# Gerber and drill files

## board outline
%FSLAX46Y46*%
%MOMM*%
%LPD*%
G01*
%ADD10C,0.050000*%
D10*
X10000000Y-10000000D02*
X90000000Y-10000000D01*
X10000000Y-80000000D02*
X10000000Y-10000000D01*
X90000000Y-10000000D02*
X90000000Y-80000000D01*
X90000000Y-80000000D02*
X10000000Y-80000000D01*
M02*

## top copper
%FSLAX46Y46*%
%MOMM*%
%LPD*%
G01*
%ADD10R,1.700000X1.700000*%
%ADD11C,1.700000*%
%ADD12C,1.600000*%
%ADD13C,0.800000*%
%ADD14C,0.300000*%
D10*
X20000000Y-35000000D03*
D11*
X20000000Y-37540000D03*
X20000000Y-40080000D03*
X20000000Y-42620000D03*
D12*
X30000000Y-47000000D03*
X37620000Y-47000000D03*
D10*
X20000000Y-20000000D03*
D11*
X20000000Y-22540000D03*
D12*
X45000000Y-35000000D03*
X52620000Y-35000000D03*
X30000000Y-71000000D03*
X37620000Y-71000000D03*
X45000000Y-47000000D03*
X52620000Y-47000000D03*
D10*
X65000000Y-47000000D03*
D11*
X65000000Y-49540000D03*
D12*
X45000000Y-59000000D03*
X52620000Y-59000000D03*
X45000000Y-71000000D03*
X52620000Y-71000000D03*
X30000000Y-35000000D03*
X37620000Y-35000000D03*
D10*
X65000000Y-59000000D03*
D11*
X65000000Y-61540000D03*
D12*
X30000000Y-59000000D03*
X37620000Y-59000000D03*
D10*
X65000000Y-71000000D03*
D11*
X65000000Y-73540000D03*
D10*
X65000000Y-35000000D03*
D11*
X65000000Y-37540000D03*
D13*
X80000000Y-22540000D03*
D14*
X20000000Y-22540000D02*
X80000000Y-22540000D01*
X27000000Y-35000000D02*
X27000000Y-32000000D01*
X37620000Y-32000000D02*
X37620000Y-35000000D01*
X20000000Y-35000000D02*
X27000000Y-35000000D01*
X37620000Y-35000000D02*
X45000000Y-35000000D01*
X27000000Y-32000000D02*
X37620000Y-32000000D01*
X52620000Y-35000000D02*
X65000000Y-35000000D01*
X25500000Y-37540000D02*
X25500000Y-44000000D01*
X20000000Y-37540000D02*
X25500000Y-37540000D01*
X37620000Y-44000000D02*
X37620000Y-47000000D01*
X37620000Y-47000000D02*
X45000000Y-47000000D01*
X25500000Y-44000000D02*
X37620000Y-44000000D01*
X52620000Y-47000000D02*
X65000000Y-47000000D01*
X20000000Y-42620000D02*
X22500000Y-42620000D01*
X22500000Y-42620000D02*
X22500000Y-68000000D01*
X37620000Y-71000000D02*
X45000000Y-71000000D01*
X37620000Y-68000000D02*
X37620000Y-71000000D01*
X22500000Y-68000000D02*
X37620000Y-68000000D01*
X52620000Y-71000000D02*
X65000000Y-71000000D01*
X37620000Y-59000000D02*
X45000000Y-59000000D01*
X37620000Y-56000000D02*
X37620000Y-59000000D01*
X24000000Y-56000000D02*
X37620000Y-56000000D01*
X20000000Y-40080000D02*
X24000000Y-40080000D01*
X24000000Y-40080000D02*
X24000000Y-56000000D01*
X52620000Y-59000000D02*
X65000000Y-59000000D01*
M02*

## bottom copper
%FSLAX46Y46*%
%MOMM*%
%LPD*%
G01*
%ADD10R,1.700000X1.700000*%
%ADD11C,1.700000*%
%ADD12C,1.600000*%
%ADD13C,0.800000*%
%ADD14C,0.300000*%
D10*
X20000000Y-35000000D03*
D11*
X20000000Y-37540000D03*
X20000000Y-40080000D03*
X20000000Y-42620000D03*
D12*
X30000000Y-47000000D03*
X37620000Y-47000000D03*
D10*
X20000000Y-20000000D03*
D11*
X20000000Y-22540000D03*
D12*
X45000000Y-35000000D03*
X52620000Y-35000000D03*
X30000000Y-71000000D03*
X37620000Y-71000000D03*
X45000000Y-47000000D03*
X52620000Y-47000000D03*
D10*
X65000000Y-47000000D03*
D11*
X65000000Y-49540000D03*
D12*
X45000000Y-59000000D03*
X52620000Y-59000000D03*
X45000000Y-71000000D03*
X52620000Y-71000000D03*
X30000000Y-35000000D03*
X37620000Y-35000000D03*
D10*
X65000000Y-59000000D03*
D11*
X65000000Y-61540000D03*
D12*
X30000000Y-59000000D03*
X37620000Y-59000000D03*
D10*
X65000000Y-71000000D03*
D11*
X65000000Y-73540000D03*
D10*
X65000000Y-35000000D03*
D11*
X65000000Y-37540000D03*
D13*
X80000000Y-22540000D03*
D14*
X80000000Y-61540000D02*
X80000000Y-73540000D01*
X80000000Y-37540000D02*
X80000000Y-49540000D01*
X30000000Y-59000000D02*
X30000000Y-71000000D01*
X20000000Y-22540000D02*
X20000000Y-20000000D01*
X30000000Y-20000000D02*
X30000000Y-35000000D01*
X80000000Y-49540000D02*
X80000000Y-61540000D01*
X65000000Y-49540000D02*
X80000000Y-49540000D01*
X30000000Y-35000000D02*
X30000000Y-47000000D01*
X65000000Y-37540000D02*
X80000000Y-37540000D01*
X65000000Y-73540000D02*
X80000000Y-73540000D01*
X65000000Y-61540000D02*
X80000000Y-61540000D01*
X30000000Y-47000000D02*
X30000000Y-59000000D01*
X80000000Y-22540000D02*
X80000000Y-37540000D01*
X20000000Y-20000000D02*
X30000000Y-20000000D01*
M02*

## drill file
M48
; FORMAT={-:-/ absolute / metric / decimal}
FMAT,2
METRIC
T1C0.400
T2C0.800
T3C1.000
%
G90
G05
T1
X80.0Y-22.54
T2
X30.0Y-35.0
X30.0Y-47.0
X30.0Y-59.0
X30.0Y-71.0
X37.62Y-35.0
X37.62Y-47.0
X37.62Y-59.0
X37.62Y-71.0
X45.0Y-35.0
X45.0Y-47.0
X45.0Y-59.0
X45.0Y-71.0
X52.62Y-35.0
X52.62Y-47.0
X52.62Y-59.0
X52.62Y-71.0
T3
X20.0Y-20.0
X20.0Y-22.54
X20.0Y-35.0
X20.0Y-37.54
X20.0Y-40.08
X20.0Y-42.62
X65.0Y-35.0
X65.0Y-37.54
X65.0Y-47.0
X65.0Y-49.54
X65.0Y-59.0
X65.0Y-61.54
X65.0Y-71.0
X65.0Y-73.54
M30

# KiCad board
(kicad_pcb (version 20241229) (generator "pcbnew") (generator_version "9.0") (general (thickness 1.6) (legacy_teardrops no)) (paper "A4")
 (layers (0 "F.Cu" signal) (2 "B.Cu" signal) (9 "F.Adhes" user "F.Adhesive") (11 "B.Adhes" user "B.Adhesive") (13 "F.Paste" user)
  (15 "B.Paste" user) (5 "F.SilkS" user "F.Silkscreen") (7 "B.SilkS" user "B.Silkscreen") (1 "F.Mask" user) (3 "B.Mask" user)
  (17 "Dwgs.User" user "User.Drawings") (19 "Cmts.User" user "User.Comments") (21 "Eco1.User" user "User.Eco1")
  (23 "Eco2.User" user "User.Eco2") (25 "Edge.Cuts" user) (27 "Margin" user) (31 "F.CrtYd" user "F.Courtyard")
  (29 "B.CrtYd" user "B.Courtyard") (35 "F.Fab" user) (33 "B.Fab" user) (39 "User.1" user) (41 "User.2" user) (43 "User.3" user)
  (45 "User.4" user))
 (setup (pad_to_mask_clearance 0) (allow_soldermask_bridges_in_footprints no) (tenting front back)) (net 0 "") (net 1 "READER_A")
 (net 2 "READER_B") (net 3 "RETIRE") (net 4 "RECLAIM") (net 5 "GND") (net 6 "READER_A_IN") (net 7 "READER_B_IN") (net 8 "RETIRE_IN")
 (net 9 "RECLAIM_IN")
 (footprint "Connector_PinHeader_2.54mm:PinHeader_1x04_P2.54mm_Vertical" (layer "F.Cu") (at 20 35)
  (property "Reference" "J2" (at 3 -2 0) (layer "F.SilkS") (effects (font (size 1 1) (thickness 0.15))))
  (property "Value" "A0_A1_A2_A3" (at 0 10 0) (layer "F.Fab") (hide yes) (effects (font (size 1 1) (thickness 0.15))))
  (pad "1" thru_hole rect (at 0 0) (size 1.7 1.7) (drill 1) (layers "*.Cu" "*.Mask") (remove_unused_layers no) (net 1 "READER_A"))
  (pad "2" thru_hole circle (at 0 2.54) (size 1.7 1.7) (drill 1) (layers "*.Cu" "*.Mask") (remove_unused_layers no) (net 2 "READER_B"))
  (pad "3" thru_hole circle (at 0 5.08) (size 1.7 1.7) (drill 1) (layers "*.Cu" "*.Mask") (remove_unused_layers no) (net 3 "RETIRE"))
  (pad "4" thru_hole circle (at 0 7.62) (size 1.7 1.7) (drill 1) (layers "*.Cu" "*.Mask") (remove_unused_layers no) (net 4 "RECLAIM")))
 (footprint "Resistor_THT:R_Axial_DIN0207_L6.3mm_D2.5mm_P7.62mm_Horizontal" (layer "F.Cu") (at 30 47)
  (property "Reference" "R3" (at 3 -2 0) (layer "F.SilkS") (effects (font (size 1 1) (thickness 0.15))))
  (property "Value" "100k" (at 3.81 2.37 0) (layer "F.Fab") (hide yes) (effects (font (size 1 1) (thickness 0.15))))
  (pad "1" thru_hole circle (at 0 0) (size 1.6 1.6) (drill 0.8) (layers "*.Cu" "*.Mask") (remove_unused_layers no) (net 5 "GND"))
  (pad "2" thru_hole circle (at 7.62 0) (size 1.6 1.6) (drill 0.8) (layers "*.Cu" "*.Mask") (remove_unused_layers no) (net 2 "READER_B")))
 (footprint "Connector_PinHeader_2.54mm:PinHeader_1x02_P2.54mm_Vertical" (layer "F.Cu") (at 20 20)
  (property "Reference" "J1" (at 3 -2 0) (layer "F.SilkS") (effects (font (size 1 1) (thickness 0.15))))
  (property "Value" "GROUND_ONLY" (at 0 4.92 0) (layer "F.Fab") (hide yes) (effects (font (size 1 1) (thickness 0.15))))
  (pad "1" thru_hole rect (at 0 0) (size 1.7 1.7) (drill 1) (layers "*.Cu" "*.Mask") (remove_unused_layers no) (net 5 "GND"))
  (pad "2" thru_hole circle (at 0 2.54) (size 1.7 1.7) (drill 1) (layers "*.Cu" "*.Mask") (remove_unused_layers no) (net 5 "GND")))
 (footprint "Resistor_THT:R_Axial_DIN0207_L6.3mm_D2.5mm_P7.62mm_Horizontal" (layer "F.Cu") (at 45 35)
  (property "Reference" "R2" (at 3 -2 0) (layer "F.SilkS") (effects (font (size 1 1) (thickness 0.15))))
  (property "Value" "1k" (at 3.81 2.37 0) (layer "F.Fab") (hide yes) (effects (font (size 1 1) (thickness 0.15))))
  (pad "1" thru_hole circle (at 0 0) (size 1.6 1.6) (drill 0.8) (layers "*.Cu" "*.Mask") (remove_unused_layers no) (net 1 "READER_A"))
  (pad "2" thru_hole circle (at 7.62 0) (size 1.6 1.6) (drill 0.8) (layers "*.Cu" "*.Mask") (remove_unused_layers no) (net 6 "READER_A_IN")))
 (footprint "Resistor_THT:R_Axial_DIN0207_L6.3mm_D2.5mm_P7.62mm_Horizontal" (layer "F.Cu") (at 30 71)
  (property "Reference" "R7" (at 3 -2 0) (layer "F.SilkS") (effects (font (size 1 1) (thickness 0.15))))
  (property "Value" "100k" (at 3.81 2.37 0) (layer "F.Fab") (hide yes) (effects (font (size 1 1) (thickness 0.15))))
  (pad "1" thru_hole circle (at 0 0) (size 1.6 1.6) (drill 0.8) (layers "*.Cu" "*.Mask") (remove_unused_layers no) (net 5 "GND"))
  (pad "2" thru_hole circle (at 7.62 0) (size 1.6 1.6) (drill 0.8) (layers "*.Cu" "*.Mask") (remove_unused_layers no) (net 4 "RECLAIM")))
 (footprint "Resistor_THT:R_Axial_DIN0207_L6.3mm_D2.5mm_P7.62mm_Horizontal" (layer "F.Cu") (at 45 47)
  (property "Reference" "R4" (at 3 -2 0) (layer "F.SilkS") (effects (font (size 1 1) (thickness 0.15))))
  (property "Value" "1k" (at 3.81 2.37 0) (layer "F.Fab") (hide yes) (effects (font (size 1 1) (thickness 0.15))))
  (pad "1" thru_hole circle (at 0 0) (size 1.6 1.6) (drill 0.8) (layers "*.Cu" "*.Mask") (remove_unused_layers no) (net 2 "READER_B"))
  (pad "2" thru_hole circle (at 7.62 0) (size 1.6 1.6) (drill 0.8) (layers "*.Cu" "*.Mask") (remove_unused_layers no) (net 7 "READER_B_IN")))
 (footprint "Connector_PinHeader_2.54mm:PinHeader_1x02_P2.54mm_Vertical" (layer "F.Cu") (at 65 47)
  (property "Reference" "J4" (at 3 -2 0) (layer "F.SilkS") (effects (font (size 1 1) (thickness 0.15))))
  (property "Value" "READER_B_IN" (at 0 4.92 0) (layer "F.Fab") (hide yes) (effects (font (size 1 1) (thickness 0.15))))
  (pad "1" thru_hole rect (at 0 0) (size 1.7 1.7) (drill 1) (layers "*.Cu" "*.Mask") (remove_unused_layers no) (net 7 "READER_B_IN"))
  (pad "2" thru_hole circle (at 0 2.54) (size 1.7 1.7) (drill 1) (layers "*.Cu" "*.Mask") (remove_unused_layers no) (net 5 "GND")))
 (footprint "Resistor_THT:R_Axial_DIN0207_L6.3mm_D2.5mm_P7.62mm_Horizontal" (layer "F.Cu") (at 45 59)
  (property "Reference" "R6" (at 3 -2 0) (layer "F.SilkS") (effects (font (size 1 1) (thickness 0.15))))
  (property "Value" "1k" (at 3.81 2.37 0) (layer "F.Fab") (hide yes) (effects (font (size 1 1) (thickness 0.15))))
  (pad "1" thru_hole circle (at 0 0) (size 1.6 1.6) (drill 0.8) (layers "*.Cu" "*.Mask") (remove_unused_layers no) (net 3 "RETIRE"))
  (pad "2" thru_hole circle (at 7.62 0) (size 1.6 1.6) (drill 0.8) (layers "*.Cu" "*.Mask") (remove_unused_layers no) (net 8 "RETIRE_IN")))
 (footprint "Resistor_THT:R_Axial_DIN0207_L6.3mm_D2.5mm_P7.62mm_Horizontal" (layer "F.Cu") (at 45 71)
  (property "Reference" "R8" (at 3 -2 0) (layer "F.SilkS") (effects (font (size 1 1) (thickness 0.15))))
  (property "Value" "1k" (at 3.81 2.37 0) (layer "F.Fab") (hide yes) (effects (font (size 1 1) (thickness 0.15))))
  (pad "1" thru_hole circle (at 0 0) (size 1.6 1.6) (drill 0.8) (layers "*.Cu" "*.Mask") (remove_unused_layers no) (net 4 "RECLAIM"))
  (pad "2" thru_hole circle (at 7.62 0) (size 1.6 1.6) (drill 0.8) (layers "*.Cu" "*.Mask") (remove_unused_layers no) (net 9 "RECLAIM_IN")))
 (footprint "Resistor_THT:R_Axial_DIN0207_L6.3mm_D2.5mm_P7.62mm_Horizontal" (layer "F.Cu") (at 30 35)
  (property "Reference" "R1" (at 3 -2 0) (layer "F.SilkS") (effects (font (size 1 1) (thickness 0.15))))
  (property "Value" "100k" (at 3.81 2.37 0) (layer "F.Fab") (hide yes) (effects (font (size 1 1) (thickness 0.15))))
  (pad "1" thru_hole circle (at 0 0) (size 1.6 1.6) (drill 0.8) (layers "*.Cu" "*.Mask") (remove_unused_layers no) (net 5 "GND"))
  (pad "2" thru_hole circle (at 7.62 0) (size 1.6 1.6) (drill 0.8) (layers "*.Cu" "*.Mask") (remove_unused_layers no) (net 1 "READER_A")))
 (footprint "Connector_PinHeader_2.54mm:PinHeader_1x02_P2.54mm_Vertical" (layer "F.Cu") (at 65 59)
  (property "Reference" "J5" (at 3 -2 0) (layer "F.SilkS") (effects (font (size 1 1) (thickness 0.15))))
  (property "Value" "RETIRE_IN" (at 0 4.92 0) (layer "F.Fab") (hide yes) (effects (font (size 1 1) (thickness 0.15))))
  (pad "1" thru_hole rect (at 0 0) (size 1.7 1.7) (drill 1) (layers "*.Cu" "*.Mask") (remove_unused_layers no) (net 8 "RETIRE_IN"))
  (pad "2" thru_hole circle (at 0 2.54) (size 1.7 1.7) (drill 1) (layers "*.Cu" "*.Mask") (remove_unused_layers no) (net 5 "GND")))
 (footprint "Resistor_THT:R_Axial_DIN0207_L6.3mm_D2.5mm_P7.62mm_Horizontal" (layer "F.Cu") (at 30 59)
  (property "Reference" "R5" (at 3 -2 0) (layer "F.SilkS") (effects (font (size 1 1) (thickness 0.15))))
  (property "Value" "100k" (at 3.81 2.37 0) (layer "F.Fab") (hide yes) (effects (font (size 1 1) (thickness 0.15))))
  (pad "1" thru_hole circle (at 0 0) (size 1.6 1.6) (drill 0.8) (layers "*.Cu" "*.Mask") (remove_unused_layers no) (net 5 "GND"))
  (pad "2" thru_hole circle (at 7.62 0) (size 1.6 1.6) (drill 0.8) (layers "*.Cu" "*.Mask") (remove_unused_layers no) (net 3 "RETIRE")))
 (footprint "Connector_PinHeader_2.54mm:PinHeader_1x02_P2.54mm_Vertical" (layer "F.Cu") (at 65 71)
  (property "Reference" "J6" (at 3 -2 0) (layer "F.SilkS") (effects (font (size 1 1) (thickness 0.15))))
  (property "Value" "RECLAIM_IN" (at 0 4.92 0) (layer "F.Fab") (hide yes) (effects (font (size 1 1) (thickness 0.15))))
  (pad "1" thru_hole rect (at 0 0) (size 1.7 1.7) (drill 1) (layers "*.Cu" "*.Mask") (remove_unused_layers no) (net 9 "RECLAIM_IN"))
  (pad "2" thru_hole circle (at 0 2.54) (size 1.7 1.7) (drill 1) (layers "*.Cu" "*.Mask") (remove_unused_layers no) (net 5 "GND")))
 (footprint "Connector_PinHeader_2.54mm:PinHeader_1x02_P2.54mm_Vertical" (layer "F.Cu") (at 65 35)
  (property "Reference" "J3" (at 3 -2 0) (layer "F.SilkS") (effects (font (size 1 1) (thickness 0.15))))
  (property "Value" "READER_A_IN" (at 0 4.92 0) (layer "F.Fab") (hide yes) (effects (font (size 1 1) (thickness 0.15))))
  (pad "1" thru_hole rect (at 0 0) (size 1.7 1.7) (drill 1) (layers "*.Cu" "*.Mask") (remove_unused_layers no) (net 6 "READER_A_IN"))
  (pad "2" thru_hole circle (at 0 2.54) (size 1.7 1.7) (drill 1) (layers "*.Cu" "*.Mask") (remove_unused_layers no) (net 5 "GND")))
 (gr_line (start 10 10) (end 90 10) (stroke (width 0.05) (type default)) (layer "Edge.Cuts"))
 (gr_line (start 10 80) (end 10 10) (stroke (width 0.05) (type default)) (layer "Edge.Cuts"))
 (gr_line (start 90 10) (end 90 80) (stroke (width 0.05) (type default)) (layer "Edge.Cuts"))
 (gr_line (start 90 80) (end 10 80) (stroke (width 0.05) (type default)) (layer "Edge.Cuts"))
 (segment (start 20 22.54) (end 80 22.54) (width 0.3) (layer "F.Cu") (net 5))
 (via (at 80 22.54) (size 0.8) (drill 0.4) (layers "F.Cu" "B.Cu") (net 5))
 (segment (start 80 61.54) (end 80 73.54) (width 0.3) (layer "B.Cu") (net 5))
 (segment (start 80 37.54) (end 80 49.54) (width 0.3) (layer "B.Cu") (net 5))
 (segment (start 30 59) (end 30 71) (width 0.3) (layer "B.Cu") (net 5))
 (segment (start 20 22.54) (end 20 20) (width 0.3) (layer "B.Cu") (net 5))
 (segment (start 30 20) (end 30 35) (width 0.3) (layer "B.Cu") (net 5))
 (segment (start 80 49.54) (end 80 61.54) (width 0.3) (layer "B.Cu") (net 5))
 (segment (start 65 49.54) (end 80 49.54) (width 0.3) (layer "B.Cu") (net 5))
 (segment (start 30 35) (end 30 47) (width 0.3) (layer "B.Cu") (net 5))
 (segment (start 65 37.54) (end 80 37.54) (width 0.3) (layer "B.Cu") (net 5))
 (segment (start 65 73.54) (end 80 73.54) (width 0.3) (layer "B.Cu") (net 5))
 (segment (start 65 61.54) (end 80 61.54) (width 0.3) (layer "B.Cu") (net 5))
 (segment (start 30 47) (end 30 59) (width 0.3) (layer "B.Cu") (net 5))
 (segment (start 80 22.54) (end 80 37.54) (width 0.3) (layer "B.Cu") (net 5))
 (segment (start 20 20) (end 30 20) (width 0.3) (layer "B.Cu") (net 5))
 (segment (start 27 35) (end 27 32) (width 0.3) (layer "F.Cu") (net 1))
 (segment (start 37.62 32) (end 37.62 35) (width 0.3) (layer "F.Cu") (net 1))
 (segment (start 20 35) (end 27 35) (width 0.3) (layer "F.Cu") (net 1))
 (segment (start 37.62 35) (end 45 35) (width 0.3) (layer "F.Cu") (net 1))
 (segment (start 27 32) (end 37.62 32) (width 0.3) (layer "F.Cu") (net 1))
 (segment (start 52.62 35) (end 65 35) (width 0.3) (layer "F.Cu") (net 6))
 (segment (start 25.5 37.54) (end 25.5 44) (width 0.3) (layer "F.Cu") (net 2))
 (segment (start 20 37.54) (end 25.5 37.54) (width 0.3) (layer "F.Cu") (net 2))
 (segment (start 37.62 44) (end 37.62 47) (width 0.3) (layer "F.Cu") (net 2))
 (segment (start 37.62 47) (end 45 47) (width 0.3) (layer "F.Cu") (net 2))
 (segment (start 25.5 44) (end 37.62 44) (width 0.3) (layer "F.Cu") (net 2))
 (segment (start 52.62 47) (end 65 47) (width 0.3) (layer "F.Cu") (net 7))
 (segment (start 20 42.62) (end 22.5 42.62) (width 0.3) (layer "F.Cu") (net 4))
 (segment (start 22.5 42.62) (end 22.5 68) (width 0.3) (layer "F.Cu") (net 4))
 (segment (start 37.62 71) (end 45 71) (width 0.3) (layer "F.Cu") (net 4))
 (segment (start 37.62 68) (end 37.62 71) (width 0.3) (layer "F.Cu") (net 4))
 (segment (start 22.5 68) (end 37.62 68) (width 0.3) (layer "F.Cu") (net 4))
 (segment (start 52.62 71) (end 65 71) (width 0.3) (layer "F.Cu") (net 9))
 (segment (start 37.62 59) (end 45 59) (width 0.3) (layer "F.Cu") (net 3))
 (segment (start 37.62 56) (end 37.62 59) (width 0.3) (layer "F.Cu") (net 3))
 (segment (start 24 56) (end 37.62 56) (width 0.3) (layer "F.Cu") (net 3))
 (segment (start 20 40.08) (end 24 40.08) (width 0.3) (layer "F.Cu") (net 3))
 (segment (start 24 40.08) (end 24 56) (width 0.3) (layer "F.Cu") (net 3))
 (segment (start 52.62 59) (end 65 59) (width 0.3) (layer "F.Cu") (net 8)))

